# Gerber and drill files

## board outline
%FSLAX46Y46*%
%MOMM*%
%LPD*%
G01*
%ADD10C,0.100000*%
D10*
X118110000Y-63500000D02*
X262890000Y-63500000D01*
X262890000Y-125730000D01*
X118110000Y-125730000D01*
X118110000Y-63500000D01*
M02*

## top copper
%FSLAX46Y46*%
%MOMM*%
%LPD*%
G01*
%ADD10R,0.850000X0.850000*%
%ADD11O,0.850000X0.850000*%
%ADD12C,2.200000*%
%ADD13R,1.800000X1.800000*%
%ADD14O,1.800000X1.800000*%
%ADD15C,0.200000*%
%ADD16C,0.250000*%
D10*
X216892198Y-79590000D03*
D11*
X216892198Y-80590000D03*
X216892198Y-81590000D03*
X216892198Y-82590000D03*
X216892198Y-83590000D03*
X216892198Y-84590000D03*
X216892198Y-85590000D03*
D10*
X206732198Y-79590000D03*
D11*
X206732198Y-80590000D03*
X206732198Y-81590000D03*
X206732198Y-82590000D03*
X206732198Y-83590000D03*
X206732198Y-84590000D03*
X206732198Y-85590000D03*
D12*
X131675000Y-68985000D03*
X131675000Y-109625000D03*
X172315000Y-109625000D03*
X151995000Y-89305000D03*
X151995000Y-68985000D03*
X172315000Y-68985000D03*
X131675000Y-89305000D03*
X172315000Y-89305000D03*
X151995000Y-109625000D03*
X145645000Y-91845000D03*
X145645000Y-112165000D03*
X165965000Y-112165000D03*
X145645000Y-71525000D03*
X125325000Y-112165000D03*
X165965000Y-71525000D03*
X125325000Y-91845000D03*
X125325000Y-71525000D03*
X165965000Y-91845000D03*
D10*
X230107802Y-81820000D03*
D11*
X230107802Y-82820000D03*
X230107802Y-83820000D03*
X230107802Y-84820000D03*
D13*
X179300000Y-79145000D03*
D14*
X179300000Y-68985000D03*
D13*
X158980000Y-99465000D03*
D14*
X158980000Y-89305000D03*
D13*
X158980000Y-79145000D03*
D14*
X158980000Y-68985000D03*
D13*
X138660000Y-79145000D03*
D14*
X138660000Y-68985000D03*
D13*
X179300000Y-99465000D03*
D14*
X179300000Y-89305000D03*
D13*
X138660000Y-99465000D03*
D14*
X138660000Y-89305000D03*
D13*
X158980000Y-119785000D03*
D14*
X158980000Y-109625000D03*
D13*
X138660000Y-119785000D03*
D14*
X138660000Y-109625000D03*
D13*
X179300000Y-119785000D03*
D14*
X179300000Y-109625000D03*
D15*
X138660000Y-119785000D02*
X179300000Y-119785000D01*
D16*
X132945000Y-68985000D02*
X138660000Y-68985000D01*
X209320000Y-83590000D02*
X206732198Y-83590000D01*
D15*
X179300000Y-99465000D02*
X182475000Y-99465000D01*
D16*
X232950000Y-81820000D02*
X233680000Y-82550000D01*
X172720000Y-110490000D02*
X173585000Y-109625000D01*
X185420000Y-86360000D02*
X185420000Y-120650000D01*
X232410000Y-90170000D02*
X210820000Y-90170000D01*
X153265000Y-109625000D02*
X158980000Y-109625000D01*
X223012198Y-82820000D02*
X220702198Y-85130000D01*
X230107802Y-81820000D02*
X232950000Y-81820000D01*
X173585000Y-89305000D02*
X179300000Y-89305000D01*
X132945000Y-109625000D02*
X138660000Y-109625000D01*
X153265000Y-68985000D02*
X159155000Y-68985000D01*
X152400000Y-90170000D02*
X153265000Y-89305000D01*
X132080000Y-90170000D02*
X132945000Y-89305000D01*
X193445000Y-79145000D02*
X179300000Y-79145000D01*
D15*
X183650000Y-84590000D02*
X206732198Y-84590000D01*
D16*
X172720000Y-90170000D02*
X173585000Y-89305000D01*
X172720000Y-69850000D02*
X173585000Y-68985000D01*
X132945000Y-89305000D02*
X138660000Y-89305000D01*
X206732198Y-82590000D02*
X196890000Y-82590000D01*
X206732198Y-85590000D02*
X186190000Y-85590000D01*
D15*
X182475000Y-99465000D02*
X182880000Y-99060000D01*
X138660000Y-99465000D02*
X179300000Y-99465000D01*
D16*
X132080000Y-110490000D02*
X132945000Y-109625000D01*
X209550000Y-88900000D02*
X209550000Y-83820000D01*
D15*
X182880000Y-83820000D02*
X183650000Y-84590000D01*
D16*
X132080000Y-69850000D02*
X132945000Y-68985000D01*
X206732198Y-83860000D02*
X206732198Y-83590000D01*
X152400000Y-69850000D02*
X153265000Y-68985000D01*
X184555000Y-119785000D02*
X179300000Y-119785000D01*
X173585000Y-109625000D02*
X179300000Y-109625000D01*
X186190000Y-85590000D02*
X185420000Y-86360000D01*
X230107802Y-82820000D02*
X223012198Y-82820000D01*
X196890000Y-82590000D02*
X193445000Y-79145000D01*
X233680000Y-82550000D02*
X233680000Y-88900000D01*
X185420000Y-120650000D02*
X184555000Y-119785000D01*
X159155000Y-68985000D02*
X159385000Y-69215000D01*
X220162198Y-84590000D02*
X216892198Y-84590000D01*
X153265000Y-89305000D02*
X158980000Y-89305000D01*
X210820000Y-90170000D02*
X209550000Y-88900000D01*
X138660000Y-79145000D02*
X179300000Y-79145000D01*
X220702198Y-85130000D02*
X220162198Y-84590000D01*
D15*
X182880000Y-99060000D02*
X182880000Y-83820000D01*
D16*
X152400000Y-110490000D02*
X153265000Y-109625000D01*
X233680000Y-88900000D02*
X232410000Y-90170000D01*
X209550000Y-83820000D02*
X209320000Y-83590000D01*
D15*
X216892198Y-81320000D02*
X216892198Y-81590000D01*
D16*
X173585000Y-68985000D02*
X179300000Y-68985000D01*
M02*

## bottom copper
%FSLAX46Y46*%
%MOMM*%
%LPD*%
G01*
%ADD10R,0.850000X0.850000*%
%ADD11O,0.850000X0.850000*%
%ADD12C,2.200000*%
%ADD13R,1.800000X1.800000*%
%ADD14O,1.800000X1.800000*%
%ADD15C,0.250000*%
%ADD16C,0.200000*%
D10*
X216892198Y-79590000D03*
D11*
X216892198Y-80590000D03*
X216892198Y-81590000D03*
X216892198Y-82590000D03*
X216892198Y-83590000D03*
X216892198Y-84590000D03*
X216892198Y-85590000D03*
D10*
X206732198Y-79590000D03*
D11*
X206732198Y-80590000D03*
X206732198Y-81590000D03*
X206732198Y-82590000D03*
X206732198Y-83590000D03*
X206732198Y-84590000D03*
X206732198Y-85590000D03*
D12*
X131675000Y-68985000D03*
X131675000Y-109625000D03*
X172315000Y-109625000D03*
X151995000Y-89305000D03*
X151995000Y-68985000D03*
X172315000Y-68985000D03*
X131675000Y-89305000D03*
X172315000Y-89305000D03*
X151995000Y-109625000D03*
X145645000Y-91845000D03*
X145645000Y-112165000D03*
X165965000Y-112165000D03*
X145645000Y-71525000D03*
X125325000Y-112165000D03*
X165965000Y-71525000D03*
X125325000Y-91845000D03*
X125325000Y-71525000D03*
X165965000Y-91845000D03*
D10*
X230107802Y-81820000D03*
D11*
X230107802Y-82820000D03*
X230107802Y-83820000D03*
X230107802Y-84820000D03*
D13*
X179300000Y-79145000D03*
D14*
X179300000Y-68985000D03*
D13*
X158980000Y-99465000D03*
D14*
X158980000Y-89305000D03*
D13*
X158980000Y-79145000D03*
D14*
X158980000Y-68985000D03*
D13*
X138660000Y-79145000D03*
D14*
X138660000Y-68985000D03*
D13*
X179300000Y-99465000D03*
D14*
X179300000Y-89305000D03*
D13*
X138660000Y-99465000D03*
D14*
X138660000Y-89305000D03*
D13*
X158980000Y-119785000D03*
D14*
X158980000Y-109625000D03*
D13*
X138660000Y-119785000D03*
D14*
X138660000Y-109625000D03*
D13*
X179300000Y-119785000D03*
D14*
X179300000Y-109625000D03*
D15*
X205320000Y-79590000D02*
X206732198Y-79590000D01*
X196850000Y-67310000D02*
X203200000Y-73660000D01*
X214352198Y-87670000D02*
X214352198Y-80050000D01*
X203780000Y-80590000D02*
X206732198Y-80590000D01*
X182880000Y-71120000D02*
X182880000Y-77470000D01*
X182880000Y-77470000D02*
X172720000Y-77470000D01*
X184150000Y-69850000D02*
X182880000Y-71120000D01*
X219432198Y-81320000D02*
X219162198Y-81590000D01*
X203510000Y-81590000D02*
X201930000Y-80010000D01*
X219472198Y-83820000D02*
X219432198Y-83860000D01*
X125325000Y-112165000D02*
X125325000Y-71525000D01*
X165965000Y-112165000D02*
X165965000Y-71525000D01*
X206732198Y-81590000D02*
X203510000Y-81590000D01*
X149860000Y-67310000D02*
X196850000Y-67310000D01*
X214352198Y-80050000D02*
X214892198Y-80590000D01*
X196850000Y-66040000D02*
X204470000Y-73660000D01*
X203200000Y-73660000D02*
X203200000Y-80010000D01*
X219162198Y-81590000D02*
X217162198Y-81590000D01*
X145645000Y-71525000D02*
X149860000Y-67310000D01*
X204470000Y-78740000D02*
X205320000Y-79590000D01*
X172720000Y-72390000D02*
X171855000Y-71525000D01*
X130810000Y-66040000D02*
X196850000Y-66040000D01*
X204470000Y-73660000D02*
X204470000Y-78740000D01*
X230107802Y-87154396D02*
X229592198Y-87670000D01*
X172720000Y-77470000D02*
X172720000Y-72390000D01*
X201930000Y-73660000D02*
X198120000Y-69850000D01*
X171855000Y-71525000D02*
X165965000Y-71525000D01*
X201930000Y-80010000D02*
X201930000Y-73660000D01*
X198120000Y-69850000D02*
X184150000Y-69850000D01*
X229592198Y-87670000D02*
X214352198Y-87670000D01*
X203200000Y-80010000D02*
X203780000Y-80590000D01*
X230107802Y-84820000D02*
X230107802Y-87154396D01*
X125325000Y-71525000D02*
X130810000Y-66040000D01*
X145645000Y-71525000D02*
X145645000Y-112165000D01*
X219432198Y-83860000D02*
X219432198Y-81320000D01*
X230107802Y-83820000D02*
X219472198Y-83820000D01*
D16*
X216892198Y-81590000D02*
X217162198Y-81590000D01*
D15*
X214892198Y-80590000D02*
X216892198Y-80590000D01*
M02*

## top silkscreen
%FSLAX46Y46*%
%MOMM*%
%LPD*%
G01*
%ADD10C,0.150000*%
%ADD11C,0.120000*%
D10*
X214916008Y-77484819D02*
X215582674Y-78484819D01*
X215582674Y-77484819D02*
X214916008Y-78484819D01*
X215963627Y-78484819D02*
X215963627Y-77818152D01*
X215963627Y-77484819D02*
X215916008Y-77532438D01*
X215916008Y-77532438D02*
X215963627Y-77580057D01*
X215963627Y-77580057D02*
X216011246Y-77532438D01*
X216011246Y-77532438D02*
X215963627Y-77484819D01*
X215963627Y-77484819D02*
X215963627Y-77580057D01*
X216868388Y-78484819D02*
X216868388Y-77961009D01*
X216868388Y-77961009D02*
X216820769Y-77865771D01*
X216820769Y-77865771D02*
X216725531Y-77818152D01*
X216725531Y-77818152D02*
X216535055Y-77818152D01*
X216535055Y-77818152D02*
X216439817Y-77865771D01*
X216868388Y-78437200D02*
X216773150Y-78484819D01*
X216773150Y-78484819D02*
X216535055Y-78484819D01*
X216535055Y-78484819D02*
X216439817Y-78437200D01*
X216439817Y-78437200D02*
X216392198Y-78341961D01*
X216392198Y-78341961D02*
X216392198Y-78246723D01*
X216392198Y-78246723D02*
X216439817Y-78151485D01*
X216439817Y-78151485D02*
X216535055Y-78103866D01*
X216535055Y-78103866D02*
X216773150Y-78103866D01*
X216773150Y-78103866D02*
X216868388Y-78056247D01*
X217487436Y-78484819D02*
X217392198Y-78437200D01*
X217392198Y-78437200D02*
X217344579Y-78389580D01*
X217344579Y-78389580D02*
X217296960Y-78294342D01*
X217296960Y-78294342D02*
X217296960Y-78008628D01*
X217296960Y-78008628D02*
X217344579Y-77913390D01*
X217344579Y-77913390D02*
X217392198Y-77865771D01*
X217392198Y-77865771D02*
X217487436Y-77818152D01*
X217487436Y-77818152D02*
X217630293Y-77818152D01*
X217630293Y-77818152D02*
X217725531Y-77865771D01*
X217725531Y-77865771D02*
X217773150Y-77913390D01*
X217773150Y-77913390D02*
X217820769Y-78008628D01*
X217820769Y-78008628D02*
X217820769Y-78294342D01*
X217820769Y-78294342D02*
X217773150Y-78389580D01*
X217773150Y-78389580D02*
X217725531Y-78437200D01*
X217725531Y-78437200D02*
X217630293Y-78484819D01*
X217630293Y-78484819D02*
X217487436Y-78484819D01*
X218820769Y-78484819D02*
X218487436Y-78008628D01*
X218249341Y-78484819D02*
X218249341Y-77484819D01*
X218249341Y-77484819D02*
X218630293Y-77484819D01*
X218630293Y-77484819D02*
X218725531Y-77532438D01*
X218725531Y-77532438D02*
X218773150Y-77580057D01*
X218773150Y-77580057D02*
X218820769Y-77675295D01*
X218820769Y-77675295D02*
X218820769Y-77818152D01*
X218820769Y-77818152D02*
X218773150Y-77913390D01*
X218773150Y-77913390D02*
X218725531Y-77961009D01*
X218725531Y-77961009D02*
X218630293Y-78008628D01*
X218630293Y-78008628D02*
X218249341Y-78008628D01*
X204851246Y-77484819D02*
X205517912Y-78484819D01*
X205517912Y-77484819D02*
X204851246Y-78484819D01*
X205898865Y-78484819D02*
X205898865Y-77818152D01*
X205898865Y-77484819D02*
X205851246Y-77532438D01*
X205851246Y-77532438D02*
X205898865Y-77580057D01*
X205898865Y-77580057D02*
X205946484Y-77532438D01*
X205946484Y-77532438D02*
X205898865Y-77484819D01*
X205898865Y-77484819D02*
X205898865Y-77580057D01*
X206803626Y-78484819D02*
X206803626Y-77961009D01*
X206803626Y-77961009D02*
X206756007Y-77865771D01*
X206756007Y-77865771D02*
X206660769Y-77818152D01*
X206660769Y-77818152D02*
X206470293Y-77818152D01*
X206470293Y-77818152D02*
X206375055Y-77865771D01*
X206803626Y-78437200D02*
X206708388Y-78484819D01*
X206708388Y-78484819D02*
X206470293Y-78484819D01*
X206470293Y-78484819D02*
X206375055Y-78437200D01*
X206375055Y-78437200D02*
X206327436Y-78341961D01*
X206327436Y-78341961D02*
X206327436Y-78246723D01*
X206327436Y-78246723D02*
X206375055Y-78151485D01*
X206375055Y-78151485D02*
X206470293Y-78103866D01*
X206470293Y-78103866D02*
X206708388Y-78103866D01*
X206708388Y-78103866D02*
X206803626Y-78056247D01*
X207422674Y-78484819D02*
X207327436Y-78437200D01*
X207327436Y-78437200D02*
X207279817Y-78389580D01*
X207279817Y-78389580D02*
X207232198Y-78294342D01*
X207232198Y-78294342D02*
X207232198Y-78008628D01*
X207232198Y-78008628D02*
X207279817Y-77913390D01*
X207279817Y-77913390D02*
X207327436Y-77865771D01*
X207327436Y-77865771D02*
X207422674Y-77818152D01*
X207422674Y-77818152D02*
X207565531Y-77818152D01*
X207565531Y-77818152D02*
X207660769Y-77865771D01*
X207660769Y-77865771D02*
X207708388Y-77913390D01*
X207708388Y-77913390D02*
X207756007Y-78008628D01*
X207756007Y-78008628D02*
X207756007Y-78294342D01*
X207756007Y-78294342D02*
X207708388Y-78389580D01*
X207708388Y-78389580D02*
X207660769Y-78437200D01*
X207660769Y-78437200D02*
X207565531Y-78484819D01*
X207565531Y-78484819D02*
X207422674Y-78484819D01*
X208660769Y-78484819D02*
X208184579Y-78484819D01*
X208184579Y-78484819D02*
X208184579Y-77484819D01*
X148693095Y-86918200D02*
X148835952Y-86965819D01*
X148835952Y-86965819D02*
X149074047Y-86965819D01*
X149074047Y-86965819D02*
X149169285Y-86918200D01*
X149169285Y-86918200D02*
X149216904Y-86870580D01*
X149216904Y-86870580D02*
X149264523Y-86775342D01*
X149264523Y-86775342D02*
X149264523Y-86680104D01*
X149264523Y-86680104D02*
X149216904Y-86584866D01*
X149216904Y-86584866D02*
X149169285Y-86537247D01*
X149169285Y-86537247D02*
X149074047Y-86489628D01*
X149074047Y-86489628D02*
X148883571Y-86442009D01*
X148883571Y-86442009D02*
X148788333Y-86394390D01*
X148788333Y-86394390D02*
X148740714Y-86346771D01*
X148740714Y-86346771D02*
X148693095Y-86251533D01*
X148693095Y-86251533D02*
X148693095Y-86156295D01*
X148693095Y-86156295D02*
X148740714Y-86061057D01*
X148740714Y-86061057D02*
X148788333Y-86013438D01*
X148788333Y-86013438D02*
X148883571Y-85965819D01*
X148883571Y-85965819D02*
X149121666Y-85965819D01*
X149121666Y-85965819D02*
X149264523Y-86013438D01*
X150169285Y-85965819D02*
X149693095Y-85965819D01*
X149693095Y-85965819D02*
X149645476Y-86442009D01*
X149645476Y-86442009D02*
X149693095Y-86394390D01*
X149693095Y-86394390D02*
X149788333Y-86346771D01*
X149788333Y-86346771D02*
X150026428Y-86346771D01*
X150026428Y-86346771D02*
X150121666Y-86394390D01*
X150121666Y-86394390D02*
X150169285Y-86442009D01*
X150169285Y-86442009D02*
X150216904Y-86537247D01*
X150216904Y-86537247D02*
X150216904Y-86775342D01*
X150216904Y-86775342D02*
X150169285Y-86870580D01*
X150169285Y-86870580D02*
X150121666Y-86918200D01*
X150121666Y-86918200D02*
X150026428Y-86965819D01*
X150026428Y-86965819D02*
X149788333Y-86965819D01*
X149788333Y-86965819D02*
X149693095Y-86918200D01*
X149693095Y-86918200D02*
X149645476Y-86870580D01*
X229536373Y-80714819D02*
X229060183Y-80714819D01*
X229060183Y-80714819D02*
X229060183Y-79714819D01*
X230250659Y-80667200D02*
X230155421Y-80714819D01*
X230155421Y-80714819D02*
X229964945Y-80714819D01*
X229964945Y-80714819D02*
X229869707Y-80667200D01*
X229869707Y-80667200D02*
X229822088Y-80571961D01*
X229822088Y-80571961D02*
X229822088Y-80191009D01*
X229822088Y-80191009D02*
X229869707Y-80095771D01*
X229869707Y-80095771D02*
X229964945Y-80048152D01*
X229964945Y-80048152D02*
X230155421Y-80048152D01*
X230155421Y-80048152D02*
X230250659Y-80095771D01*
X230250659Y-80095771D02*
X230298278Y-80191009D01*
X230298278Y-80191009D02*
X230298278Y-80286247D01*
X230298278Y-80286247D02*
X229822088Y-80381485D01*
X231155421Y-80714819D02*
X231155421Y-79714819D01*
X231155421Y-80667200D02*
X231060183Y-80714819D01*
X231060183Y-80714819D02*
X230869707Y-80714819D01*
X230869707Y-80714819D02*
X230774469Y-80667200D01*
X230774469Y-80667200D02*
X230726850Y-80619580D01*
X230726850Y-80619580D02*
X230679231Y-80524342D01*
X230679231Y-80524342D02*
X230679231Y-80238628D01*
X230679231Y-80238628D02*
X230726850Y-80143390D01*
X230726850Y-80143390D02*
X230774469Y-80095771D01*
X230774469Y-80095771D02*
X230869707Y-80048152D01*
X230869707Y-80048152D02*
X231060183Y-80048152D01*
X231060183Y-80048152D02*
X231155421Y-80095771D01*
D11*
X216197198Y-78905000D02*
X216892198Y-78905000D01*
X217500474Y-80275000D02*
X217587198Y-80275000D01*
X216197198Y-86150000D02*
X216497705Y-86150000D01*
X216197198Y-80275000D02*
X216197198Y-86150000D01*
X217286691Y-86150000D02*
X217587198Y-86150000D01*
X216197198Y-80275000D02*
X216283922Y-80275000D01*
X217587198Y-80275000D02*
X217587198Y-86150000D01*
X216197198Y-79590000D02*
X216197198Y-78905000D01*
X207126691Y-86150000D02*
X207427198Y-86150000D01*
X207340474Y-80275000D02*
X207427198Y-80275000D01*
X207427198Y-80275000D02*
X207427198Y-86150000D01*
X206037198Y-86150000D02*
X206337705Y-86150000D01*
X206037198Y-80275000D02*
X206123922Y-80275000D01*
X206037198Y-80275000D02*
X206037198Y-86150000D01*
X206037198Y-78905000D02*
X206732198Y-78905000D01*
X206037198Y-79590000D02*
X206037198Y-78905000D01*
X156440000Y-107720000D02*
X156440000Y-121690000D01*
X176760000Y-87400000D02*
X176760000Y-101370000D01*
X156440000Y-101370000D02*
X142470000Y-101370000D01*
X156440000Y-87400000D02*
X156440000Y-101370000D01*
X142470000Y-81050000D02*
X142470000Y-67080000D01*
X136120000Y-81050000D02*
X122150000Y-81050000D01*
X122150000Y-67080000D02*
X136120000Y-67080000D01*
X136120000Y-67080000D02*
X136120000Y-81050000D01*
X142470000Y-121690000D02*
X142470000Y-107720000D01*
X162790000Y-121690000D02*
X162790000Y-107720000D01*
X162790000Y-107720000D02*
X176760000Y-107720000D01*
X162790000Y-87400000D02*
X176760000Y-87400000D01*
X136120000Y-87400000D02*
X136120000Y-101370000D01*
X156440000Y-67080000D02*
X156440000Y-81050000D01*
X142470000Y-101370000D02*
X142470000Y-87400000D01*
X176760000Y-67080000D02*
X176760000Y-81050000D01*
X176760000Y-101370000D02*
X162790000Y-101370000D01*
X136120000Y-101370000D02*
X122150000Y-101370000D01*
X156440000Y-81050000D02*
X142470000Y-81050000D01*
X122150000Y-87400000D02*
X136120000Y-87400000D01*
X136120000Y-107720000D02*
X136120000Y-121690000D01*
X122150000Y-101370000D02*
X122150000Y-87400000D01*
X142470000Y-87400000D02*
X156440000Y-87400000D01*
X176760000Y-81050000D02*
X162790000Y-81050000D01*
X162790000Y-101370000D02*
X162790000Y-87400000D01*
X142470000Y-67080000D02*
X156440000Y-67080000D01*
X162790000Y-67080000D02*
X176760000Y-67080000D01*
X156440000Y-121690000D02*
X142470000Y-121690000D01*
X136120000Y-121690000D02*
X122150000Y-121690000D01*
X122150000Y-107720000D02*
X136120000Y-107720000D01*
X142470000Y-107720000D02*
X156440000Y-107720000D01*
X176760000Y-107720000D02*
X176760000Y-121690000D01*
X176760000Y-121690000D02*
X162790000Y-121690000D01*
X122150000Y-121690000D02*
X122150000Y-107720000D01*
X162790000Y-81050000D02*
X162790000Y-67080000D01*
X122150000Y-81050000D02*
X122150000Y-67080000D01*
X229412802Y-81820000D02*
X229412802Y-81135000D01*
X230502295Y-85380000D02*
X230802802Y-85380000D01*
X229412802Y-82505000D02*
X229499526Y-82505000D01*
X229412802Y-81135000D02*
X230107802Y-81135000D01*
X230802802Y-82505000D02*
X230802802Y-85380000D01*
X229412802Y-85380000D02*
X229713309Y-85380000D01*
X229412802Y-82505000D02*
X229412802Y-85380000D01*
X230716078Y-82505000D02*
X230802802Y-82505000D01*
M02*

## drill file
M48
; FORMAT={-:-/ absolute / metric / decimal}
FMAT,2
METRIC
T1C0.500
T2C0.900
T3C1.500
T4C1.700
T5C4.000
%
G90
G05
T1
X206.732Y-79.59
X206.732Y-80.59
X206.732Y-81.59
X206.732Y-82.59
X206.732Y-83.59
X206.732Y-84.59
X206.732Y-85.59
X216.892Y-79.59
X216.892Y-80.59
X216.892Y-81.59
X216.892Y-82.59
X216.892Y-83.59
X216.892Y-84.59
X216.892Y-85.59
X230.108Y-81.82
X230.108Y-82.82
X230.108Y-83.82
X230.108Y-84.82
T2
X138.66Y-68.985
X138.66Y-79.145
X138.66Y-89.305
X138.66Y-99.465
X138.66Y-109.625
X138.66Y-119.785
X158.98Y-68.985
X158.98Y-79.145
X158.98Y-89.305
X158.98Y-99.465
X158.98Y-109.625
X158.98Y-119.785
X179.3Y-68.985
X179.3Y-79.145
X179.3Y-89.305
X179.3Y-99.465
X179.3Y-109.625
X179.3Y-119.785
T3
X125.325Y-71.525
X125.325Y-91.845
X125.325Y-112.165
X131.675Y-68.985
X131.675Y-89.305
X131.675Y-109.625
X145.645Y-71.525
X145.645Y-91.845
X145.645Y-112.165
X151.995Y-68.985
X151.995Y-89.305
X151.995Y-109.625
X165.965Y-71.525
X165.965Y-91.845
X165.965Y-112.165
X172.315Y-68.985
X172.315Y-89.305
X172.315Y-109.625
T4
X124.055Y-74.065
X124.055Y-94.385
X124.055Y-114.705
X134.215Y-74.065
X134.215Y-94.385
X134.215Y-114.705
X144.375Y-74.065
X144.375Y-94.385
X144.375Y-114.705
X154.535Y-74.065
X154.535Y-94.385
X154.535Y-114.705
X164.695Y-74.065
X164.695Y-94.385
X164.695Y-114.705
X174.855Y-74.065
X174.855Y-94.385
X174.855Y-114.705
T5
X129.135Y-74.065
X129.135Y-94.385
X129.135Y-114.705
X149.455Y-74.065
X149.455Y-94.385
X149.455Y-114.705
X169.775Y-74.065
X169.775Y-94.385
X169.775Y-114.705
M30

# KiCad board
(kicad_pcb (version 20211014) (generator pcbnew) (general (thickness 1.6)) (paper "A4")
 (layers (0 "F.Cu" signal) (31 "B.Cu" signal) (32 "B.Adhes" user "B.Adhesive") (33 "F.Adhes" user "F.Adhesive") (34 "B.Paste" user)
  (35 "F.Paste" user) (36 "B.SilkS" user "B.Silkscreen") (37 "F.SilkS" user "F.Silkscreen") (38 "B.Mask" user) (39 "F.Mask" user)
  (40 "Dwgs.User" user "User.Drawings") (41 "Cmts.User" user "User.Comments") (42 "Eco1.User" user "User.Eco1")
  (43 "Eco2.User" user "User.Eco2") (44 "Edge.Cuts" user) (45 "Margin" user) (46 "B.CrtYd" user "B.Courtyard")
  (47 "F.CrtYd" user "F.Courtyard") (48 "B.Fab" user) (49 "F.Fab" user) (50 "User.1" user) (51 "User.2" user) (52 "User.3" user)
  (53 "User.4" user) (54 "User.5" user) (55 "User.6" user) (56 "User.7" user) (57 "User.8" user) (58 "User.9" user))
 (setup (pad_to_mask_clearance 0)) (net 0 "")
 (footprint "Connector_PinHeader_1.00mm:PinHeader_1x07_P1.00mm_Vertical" (layer "F.Cu") (at 216.892198 79.59)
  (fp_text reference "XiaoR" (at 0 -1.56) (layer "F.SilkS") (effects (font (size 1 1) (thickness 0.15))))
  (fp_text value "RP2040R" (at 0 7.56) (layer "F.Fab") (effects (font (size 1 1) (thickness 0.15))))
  (fp_line (start -0.695 -0.685) (end 0 -0.685) (layer "F.SilkS") (width 0.12))
  (fp_line (start 0.608276 0.685) (end 0.695 0.685) (layer "F.SilkS") (width 0.12))
  (fp_line (start -0.695 6.56) (end -0.394493 6.56) (layer "F.SilkS") (width 0.12))
  (fp_line (start -0.695 0.685) (end -0.695 6.56) (layer "F.SilkS") (width 0.12))
  (fp_line (start 0.394493 6.56) (end 0.695 6.56) (layer "F.SilkS") (width 0.12))
  (fp_line (start -0.695 0.685) (end -0.608276 0.685) (layer "F.SilkS") (width 0.12))
  (fp_line (start 0.695 0.685) (end 0.695 6.56) (layer "F.SilkS") (width 0.12))
  (fp_line (start -0.695 0) (end -0.695 -0.685) (layer "F.SilkS") (width 0.12))
  (pad "1" thru_hole rect (at 0 0) (size 0.85 0.85) (drill 0.5) (layers F&B.Cu *.Mask))
  (pad "2" thru_hole oval (at 0 1) (size 0.85 0.85) (drill 0.5) (layers F&B.Cu *.Mask))
  (pad "3" thru_hole oval (at 0 2) (size 0.85 0.85) (drill 0.5) (layers F&B.Cu *.Mask))
  (pad "4" thru_hole oval (at 0 3) (size 0.85 0.85) (drill 0.5) (layers F&B.Cu *.Mask))
  (pad "5" thru_hole oval (at 0 4) (size 0.85 0.85) (drill 0.5) (layers F&B.Cu *.Mask))
  (pad "6" thru_hole oval (at 0 5) (size 0.85 0.85) (drill 0.5) (layers F&B.Cu *.Mask))
  (pad "7" thru_hole oval (at 0 6) (size 0.85 0.85) (drill 0.5) (layers F&B.Cu *.Mask)))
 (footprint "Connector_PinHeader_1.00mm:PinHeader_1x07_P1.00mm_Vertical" (layer "F.Cu") (at 206.732198 79.59)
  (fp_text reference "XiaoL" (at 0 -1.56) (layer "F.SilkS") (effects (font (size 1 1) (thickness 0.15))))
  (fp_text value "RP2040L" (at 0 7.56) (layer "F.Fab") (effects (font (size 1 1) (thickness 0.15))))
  (fp_line (start 0.394493 6.56) (end 0.695 6.56) (layer "F.SilkS") (width 0.12))
  (fp_line (start 0.608276 0.685) (end 0.695 0.685) (layer "F.SilkS") (width 0.12))
  (fp_line (start 0.695 0.685) (end 0.695 6.56) (layer "F.SilkS") (width 0.12))
  (fp_line (start -0.695 6.56) (end -0.394493 6.56) (layer "F.SilkS") (width 0.12))
  (fp_line (start -0.695 0.685) (end -0.608276 0.685) (layer "F.SilkS") (width 0.12))
  (fp_line (start -0.695 0.685) (end -0.695 6.56) (layer "F.SilkS") (width 0.12))
  (fp_line (start -0.695 -0.685) (end 0 -0.685) (layer "F.SilkS") (width 0.12))
  (fp_line (start -0.695 0) (end -0.695 -0.685) (layer "F.SilkS") (width 0.12))
  (pad "1" thru_hole rect (at 0 0) (size 0.85 0.85) (drill 0.5) (layers *.Cu *.Mask))
  (pad "2" thru_hole oval (at 0 1) (size 0.85 0.85) (drill 0.5) (layers *.Cu *.Mask))
  (pad "3" thru_hole oval (at 0 2) (size 0.85 0.85) (drill 0.5) (layers *.Cu *.Mask))
  (pad "4" thru_hole oval (at 0 3) (size 0.85 0.85) (drill 0.5) (layers *.Cu *.Mask))
  (pad "5" thru_hole oval (at 0 4) (size 0.85 0.85) (drill 0.5) (layers *.Cu *.Mask))
  (pad "6" thru_hole oval (at 0 5) (size 0.85 0.85) (drill 0.5) (layers *.Cu *.Mask))
  (pad "7" thru_hole oval (at 0 6) (size 0.85 0.85) (drill 0.5) (layers *.Cu *.Mask)))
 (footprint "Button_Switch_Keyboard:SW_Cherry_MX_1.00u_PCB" (layer "F.Cu") (at 276.455 61.365)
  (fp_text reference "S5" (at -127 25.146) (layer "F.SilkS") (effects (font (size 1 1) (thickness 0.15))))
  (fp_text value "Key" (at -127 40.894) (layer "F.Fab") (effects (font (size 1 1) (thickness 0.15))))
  (fp_line (start -120.015 46.355) (end -120.015 60.325) (layer "F.SilkS") (width 0.12))
  (fp_line (start -99.695 26.035) (end -99.695 40.005) (layer "F.SilkS") (width 0.12))
  (fp_line (start -120.015 40.005) (end -133.985 40.005) (layer "F.SilkS") (width 0.12))
  (fp_line (start -120.015 26.035) (end -120.015 40.005) (layer "F.SilkS") (width 0.12))
  (fp_line (start -133.985 19.685) (end -133.985 5.715) (layer "F.SilkS") (width 0.12))
  (fp_line (start -140.335 19.685) (end -154.305 19.685) (layer "F.SilkS") (width 0.12))
  (fp_line (start -154.305 5.715) (end -140.335 5.715) (layer "F.SilkS") (width 0.12))
  (fp_line (start -140.335 5.715) (end -140.335 19.685) (layer "F.SilkS") (width 0.12))
  (fp_line (start -133.985 60.325) (end -133.985 46.355) (layer "F.SilkS") (width 0.12))
  (fp_line (start -113.665 60.325) (end -113.665 46.355) (layer "F.SilkS") (width 0.12))
  (fp_line (start -113.665 46.355) (end -99.695 46.355) (layer "F.SilkS") (width 0.12))
  (fp_line (start -113.665 26.035) (end -99.695 26.035) (layer "F.SilkS") (width 0.12))
  (fp_line (start -140.335 26.035) (end -140.335 40.005) (layer "F.SilkS") (width 0.12))
  (fp_line (start -120.015 5.715) (end -120.015 19.685) (layer "F.SilkS") (width 0.12))
  (fp_line (start -133.985 40.005) (end -133.985 26.035) (layer "F.SilkS") (width 0.12))
  (fp_line (start -99.695 5.715) (end -99.695 19.685) (layer "F.SilkS") (width 0.12))
  (fp_line (start -99.695 40.005) (end -113.665 40.005) (layer "F.SilkS") (width 0.12))
  (fp_line (start -140.335 40.005) (end -154.305 40.005) (layer "F.SilkS") (width 0.12))
  (fp_line (start -120.015 19.685) (end -133.985 19.685) (layer "F.SilkS") (width 0.12))
  (fp_line (start -154.305 26.035) (end -140.335 26.035) (layer "F.SilkS") (width 0.12))
  (fp_line (start -140.335 46.355) (end -140.335 60.325) (layer "F.SilkS") (width 0.12))
  (fp_line (start -154.305 40.005) (end -154.305 26.035) (layer "F.SilkS") (width 0.12))
  (fp_line (start -133.985 26.035) (end -120.015 26.035) (layer "F.SilkS") (width 0.12))
  (fp_line (start -99.695 19.685) (end -113.665 19.685) (layer "F.SilkS") (width 0.12))
  (fp_line (start -113.665 40.005) (end -113.665 26.035) (layer "F.SilkS") (width 0.12))
  (fp_line (start -133.985 5.715) (end -120.015 5.715) (layer "F.SilkS") (width 0.12))
  (fp_line (start -113.665 5.715) (end -99.695 5.715) (layer "F.SilkS") (width 0.12))
  (fp_line (start -120.015 60.325) (end -133.985 60.325) (layer "F.SilkS") (width 0.12))
  (fp_line (start -140.335 60.325) (end -154.305 60.325) (layer "F.SilkS") (width 0.12))
  (fp_line (start -154.305 46.355) (end -140.335 46.355) (layer "F.SilkS") (width 0.12))
  (fp_line (start -133.985 46.355) (end -120.015 46.355) (layer "F.SilkS") (width 0.12))
  (fp_line (start -99.695 46.355) (end -99.695 60.325) (layer "F.SilkS") (width 0.12))
  (fp_line (start -99.695 60.325) (end -113.665 60.325) (layer "F.SilkS") (width 0.12))
  (fp_line (start -154.305 60.325) (end -154.305 46.355) (layer "F.SilkS") (width 0.12))
  (fp_line (start -113.665 19.685) (end -113.665 5.715) (layer "F.SilkS") (width 0.12))
  (fp_line (start -154.305 19.685) (end -154.305 5.715) (layer "F.SilkS") (width 0.12))
  (pad "" np_thru_hole circle (at -152.4 33.02) (size 1.7 1.7) (drill 1.7) (layers *.Cu *.Mask))
  (pad "" np_thru_hole circle (at -121.92 53.34) (size 1.7 1.7) (drill 1.7) (layers *.Cu *.Mask))
  (pad "" np_thru_hole circle (at -132.08 12.7) (size 1.7 1.7) (drill 1.7) (layers *.Cu *.Mask))
  (pad "" np_thru_hole circle (at -127 33.02) (size 4 4) (drill 4) (layers *.Cu *.Mask))
  (pad "" np_thru_hole circle (at -142.24 12.7) (size 1.7 1.7) (drill 1.7) (layers *.Cu *.Mask))
  (pad "" np_thru_hole circle (at -147.32 53.34) (size 4 4) (drill 4) (layers *.Cu *.Mask))
  (pad "" np_thru_hole circle (at -152.4 12.7) (size 1.7 1.7) (drill 1.7) (layers *.Cu *.Mask))
  (pad "" np_thru_hole circle (at -106.68 12.7) (size 4 4) (drill 4) (layers *.Cu *.Mask))
  (pad "" np_thru_hole circle (at -142.24 33.02) (size 1.7 1.7) (drill 1.7) (layers *.Cu *.Mask))
  (pad "" np_thru_hole circle (at -127 53.34) (size 4 4) (drill 4) (layers *.Cu *.Mask))
  (pad "" np_thru_hole circle (at -111.76 53.34) (size 1.7 1.7) (drill 1.7) (layers *.Cu *.Mask))
  (pad "" np_thru_hole circle (at -127 12.7) (size 4 4) (drill 4) (layers *.Cu *.Mask))
  (pad "" np_thru_hole circle (at -142.24 53.34) (size 1.7 1.7) (drill 1.7) (layers *.Cu *.Mask))
  (pad "" np_thru_hole circle (at -147.32 12.7) (size 4 4) (drill 4) (layers *.Cu *.Mask))
  (pad "" np_thru_hole circle (at -132.08 53.34) (size 1.7 1.7) (drill 1.7) (layers *.Cu *.Mask))
  (pad "" np_thru_hole circle (at -101.6 53.34) (size 1.7 1.7) (drill 1.7) (layers *.Cu *.Mask))
  (pad "" np_thru_hole circle (at -106.68 33.02) (size 4 4) (drill 4) (layers *.Cu *.Mask))
  (pad "" np_thru_hole circle (at -101.6 33.02) (size 1.7 1.7) (drill 1.7) (layers *.Cu *.Mask))
  (pad "" np_thru_hole circle (at -101.6 12.7) (size 1.7 1.7) (drill 1.7) (layers *.Cu *.Mask))
  (pad "" np_thru_hole circle (at -121.92 12.7) (size 1.7 1.7) (drill 1.7) (layers *.Cu *.Mask))
  (pad "" np_thru_hole circle (at -111.76 33.02) (size 1.7 1.7) (drill 1.7) (layers *.Cu *.Mask))
  (pad "" np_thru_hole circle (at -121.92 33.02) (size 1.7 1.7) (drill 1.7) (layers *.Cu *.Mask))
  (pad "" np_thru_hole circle (at -106.68 53.34) (size 4 4) (drill 4) (layers *.Cu *.Mask))
  (pad "" np_thru_hole circle (at -152.4 53.34) (size 1.7 1.7) (drill 1.7) (layers *.Cu *.Mask))
  (pad "" np_thru_hole circle (at -111.76 12.7) (size 1.7 1.7) (drill 1.7) (layers *.Cu *.Mask))
  (pad "" np_thru_hole circle (at -147.32 33.02) (size 4 4) (drill 4) (layers *.Cu *.Mask))
  (pad "" np_thru_hole circle (at -132.08 33.02) (size 1.7 1.7) (drill 1.7) (layers *.Cu *.Mask))
  (pad "1" thru_hole circle (at -144.78 7.62) (size 2.2 2.2) (drill 1.5) (layers *.Cu *.Mask))
  (pad "1" thru_hole circle (at -144.78 48.26) (size 2.2 2.2) (drill 1.5) (layers *.Cu *.Mask))
  (pad "1" thru_hole circle (at -104.14 48.26) (size 2.2 2.2) (drill 1.5) (layers *.Cu *.Mask))
  (pad "1" thru_hole circle (at -124.46 27.94) (size 2.2 2.2) (drill 1.5) (layers *.Cu *.Mask))
  (pad "1" thru_hole circle (at -124.46 7.62) (size 2.2 2.2) (drill 1.5) (layers *.Cu *.Mask))
  (pad "1" thru_hole circle (at -104.14 7.62) (size 2.2 2.2) (drill 1.5) (layers *.Cu *.Mask))
  (pad "1" thru_hole circle (at -144.78 27.94) (size 2.2 2.2) (drill 1.5) (layers *.Cu *.Mask))
  (pad "1" thru_hole circle (at -104.14 27.94) (size 2.2 2.2) (drill 1.5) (layers *.Cu *.Mask))
  (pad "1" thru_hole circle (at -124.46 48.26) (size 2.2 2.2) (drill 1.5) (layers *.Cu *.Mask))
  (pad "2" thru_hole circle (at -130.81 30.48) (size 2.2 2.2) (drill 1.5) (layers *.Cu *.Mask))
  (pad "2" thru_hole circle (at -130.81 50.8) (size 2.2 2.2) (drill 1.5) (layers *.Cu *.Mask))
  (pad "2" thru_hole circle (at -110.49 50.8) (size 2.2 2.2) (drill 1.5) (layers *.Cu *.Mask))
  (pad "2" thru_hole circle (at -130.81 10.16) (size 2.2 2.2) (drill 1.5) (layers *.Cu *.Mask))
  (pad "2" thru_hole circle (at -151.13 50.8) (size 2.2 2.2) (drill 1.5) (layers *.Cu *.Mask))
  (pad "2" thru_hole circle (at -110.49 10.16) (size 2.2 2.2) (drill 1.5) (layers *.Cu *.Mask))
  (pad "2" thru_hole circle (at -151.13 30.48) (size 2.2 2.2) (drill 1.5) (layers *.Cu *.Mask))
  (pad "2" thru_hole circle (at -151.13 10.16) (size 2.2 2.2) (drill 1.5) (layers *.Cu *.Mask))
  (pad "2" thru_hole circle (at -110.49 30.48) (size 2.2 2.2) (drill 1.5) (layers *.Cu *.Mask)))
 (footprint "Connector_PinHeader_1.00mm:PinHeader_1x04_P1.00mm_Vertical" (layer "F.Cu") (at 230.107802 81.82)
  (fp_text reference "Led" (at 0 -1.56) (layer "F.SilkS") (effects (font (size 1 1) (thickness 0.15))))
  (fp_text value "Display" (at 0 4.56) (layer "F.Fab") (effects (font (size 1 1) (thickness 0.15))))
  (fp_line (start -0.695 0) (end -0.695 -0.685) (layer "F.SilkS") (width 0.12))
  (fp_line (start 0.394493 3.56) (end 0.695 3.56) (layer "F.SilkS") (width 0.12))
  (fp_line (start -0.695 0.685) (end -0.608276 0.685) (layer "F.SilkS") (width 0.12))
  (fp_line (start -0.695 -0.685) (end 0 -0.685) (layer "F.SilkS") (width 0.12))
  (fp_line (start 0.695 0.685) (end 0.695 3.56) (layer "F.SilkS") (width 0.12))
  (fp_line (start -0.695 3.56) (end -0.394493 3.56) (layer "F.SilkS") (width 0.12))
  (fp_line (start -0.695 0.685) (end -0.695 3.56) (layer "F.SilkS") (width 0.12))
  (fp_line (start 0.608276 0.685) (end 0.695 0.685) (layer "F.SilkS") (width 0.12))
  (pad "1" thru_hole rect (at 0 0) (size 0.85 0.85) (drill 0.5) (layers *.Cu *.Mask))
  (pad "2" thru_hole oval (at 0 1) (size 0.85 0.85) (drill 0.5) (layers *.Cu *.Mask))
  (pad "3" thru_hole oval (at 0 2) (size 0.85 0.85) (drill 0.5) (layers *.Cu *.Mask))
  (pad "4" thru_hole oval (at 0 3) (size 0.85 0.85) (drill 0.5) (layers *.Cu *.Mask)))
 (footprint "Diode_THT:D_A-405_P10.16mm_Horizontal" (layer "B.Cu") (at 179.3 79.145 90)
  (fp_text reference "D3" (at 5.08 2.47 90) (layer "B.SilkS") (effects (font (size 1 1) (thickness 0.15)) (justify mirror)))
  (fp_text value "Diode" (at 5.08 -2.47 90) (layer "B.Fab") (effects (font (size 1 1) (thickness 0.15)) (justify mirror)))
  (pad "1" thru_hole rect (at 0 0 90) (size 1.8 1.8) (drill 0.9) (layers F&B.Cu *.Mask))
  (pad "2" thru_hole oval (at 10.16 0 90) (size 1.8 1.8) (drill 0.9) (layers F&B.Cu *.Mask)))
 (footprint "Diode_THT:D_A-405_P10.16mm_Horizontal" (layer "B.Cu") (at 158.98 99.465 90)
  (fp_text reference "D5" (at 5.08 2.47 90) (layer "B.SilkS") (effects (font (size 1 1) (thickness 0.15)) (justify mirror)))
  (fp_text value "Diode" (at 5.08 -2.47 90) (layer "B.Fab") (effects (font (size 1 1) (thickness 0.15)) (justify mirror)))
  (pad "1" thru_hole rect (at 0 0 90) (size 1.8 1.8) (drill 0.9) (layers F&B.Cu *.Mask))
  (pad "2" thru_hole oval (at 10.16 0 90) (size 1.8 1.8) (drill 0.9) (layers F&B.Cu *.Mask)))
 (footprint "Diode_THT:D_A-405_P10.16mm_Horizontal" (layer "B.Cu") (at 158.98 79.145 90)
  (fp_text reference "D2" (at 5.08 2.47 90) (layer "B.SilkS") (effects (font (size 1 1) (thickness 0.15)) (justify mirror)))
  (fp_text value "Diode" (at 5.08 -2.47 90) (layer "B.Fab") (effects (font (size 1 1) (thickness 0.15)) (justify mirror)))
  (pad "1" thru_hole rect (at 0 0 90) (size 1.8 1.8) (drill 0.9) (layers F&B.Cu *.Mask))
  (pad "2" thru_hole oval (at 10.16 0 90) (size 1.8 1.8) (drill 0.9) (layers F&B.Cu *.Mask)))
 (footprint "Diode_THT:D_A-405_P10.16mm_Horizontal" (layer "B.Cu") (at 138.66 79.145 90)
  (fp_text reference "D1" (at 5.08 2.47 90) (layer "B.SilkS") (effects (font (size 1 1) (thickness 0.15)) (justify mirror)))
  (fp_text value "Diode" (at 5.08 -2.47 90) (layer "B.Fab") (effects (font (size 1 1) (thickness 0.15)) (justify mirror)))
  (pad "1" thru_hole rect (at 0 0 90) (size 1.8 1.8) (drill 0.9) (layers *.Cu *.Mask))
  (pad "2" thru_hole oval (at 10.16 0 90) (size 1.8 1.8) (drill 0.9) (layers *.Cu *.Mask)))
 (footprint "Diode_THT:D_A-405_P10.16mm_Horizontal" (layer "B.Cu") (at 179.3 99.465 90)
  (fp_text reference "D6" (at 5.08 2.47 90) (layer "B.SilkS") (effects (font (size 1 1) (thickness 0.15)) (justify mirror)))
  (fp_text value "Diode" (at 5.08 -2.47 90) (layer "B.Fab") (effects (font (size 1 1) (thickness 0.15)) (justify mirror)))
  (pad "1" thru_hole rect (at 0 0 90) (size 1.8 1.8) (drill 0.9) (layers F&B.Cu *.Mask))
  (pad "2" thru_hole oval (at 10.16 0 90) (size 1.8 1.8) (drill 0.9) (layers F&B.Cu *.Mask)))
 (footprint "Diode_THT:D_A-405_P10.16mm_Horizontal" (layer "B.Cu") (at 138.66 99.465 90)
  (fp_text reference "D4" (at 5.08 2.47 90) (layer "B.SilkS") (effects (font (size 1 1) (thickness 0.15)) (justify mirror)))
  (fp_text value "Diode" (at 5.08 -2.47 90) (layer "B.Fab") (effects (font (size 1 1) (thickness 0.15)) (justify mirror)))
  (pad "1" thru_hole rect (at 0 0 90) (size 1.8 1.8) (drill 0.9) (layers F&B.Cu *.Mask))
  (pad "2" thru_hole oval (at 10.16 0 90) (size 1.8 1.8) (drill 0.9) (layers F&B.Cu *.Mask)))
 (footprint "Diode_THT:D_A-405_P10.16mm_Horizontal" (layer "B.Cu") (at 158.98 119.785 90)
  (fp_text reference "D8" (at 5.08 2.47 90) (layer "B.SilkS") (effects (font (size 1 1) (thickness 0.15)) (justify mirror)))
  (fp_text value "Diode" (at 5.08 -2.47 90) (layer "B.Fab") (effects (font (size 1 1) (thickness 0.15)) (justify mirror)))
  (pad "1" thru_hole rect (at 0 0 90) (size 1.8 1.8) (drill 0.9) (layers F&B.Cu *.Mask))
  (pad "2" thru_hole oval (at 10.16 0 90) (size 1.8 1.8) (drill 0.9) (layers F&B.Cu *.Mask)))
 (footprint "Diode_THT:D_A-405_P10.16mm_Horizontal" (layer "B.Cu") (at 138.66 119.785 90)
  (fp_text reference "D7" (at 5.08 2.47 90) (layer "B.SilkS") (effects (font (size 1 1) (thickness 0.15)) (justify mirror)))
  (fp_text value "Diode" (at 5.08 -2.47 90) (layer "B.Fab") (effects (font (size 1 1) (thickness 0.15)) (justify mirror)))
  (pad "1" thru_hole rect (at 0 0 90) (size 1.8 1.8) (drill 0.9) (layers F&B.Cu *.Mask))
  (pad "2" thru_hole oval (at 10.16 0 90) (size 1.8 1.8) (drill 0.9) (layers F&B.Cu *.Mask)))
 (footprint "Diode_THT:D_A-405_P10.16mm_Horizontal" (layer "B.Cu") (at 179.3 119.785 90)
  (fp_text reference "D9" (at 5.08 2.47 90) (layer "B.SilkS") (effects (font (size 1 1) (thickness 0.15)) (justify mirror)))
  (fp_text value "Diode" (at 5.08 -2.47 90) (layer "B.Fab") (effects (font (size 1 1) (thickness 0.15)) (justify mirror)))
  (pad "1" thru_hole rect (at 0 0 90) (size 1.8 1.8) (drill 0.9) (layers F&B.Cu *.Mask))
  (pad "2" thru_hole oval (at 10.16 0 90) (size 1.8 1.8) (drill 0.9) (layers F&B.Cu *.Mask)))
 (gr_rect (start 262.89 125.73) (end 118.11 63.5) (layer "Edge.Cuts") (width 0.1) (fill none))
 (segment (start 138.66 119.785) (end 179.3 119.785) (width 0.2) (layer "F.Cu") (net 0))
 (segment (start 132.945 68.985) (end 138.66 68.985) (width 0.25) (layer "F.Cu") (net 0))
 (segment (start 209.32 83.59) (end 206.732198 83.59) (width 0.25) (layer "F.Cu") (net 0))
 (segment (start 179.3 99.465) (end 182.475 99.465) (width 0.2) (layer "F.Cu") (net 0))
 (segment (start 232.95 81.82) (end 233.68 82.55) (width 0.25) (layer "F.Cu") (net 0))
 (segment (start 172.72 110.49) (end 173.585 109.625) (width 0.25) (layer "F.Cu") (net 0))
 (segment (start 185.42 86.36) (end 185.42 120.65) (width 0.25) (layer "F.Cu") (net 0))
 (segment (start 232.41 90.17) (end 210.82 90.17) (width 0.25) (layer "F.Cu") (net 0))
 (segment (start 153.265 109.625) (end 158.98 109.625) (width 0.25) (layer "F.Cu") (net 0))
 (segment (start 223.012198 82.82) (end 220.702198 85.13) (width 0.25) (layer "F.Cu") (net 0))
 (segment (start 230.107802 81.82) (end 232.95 81.82) (width 0.25) (layer "F.Cu") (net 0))
 (segment (start 173.585 89.305) (end 179.3 89.305) (width 0.25) (layer "F.Cu") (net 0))
 (segment (start 132.945 109.625) (end 138.66 109.625) (width 0.25) (layer "F.Cu") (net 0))
 (segment (start 153.265 68.985) (end 159.155 68.985) (width 0.25) (layer "F.Cu") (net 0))
 (segment (start 152.4 90.17) (end 153.265 89.305) (width 0.25) (layer "F.Cu") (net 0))
 (segment (start 132.08 90.17) (end 132.945 89.305) (width 0.25) (layer "F.Cu") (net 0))
 (segment (start 193.445 79.145) (end 179.3 79.145) (width 0.25) (layer "F.Cu") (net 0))
 (segment (start 183.65 84.59) (end 206.732198 84.59) (width 0.2) (layer "F.Cu") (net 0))
 (segment (start 172.72 90.17) (end 173.585 89.305) (width 0.25) (layer "F.Cu") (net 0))
 (segment (start 172.72 69.85) (end 173.585 68.985) (width 0.25) (layer "F.Cu") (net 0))
 (segment (start 132.945 89.305) (end 138.66 89.305) (width 0.25) (layer "F.Cu") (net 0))
 (segment (start 206.732198 82.59) (end 196.89 82.59) (width 0.25) (layer "F.Cu") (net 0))
 (segment (start 206.732198 85.59) (end 186.19 85.59) (width 0.25) (layer "F.Cu") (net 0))
 (segment (start 182.475 99.465) (end 182.88 99.06) (width 0.2) (layer "F.Cu") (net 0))
 (segment (start 138.66 99.465) (end 179.3 99.465) (width 0.2) (layer "F.Cu") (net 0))
 (segment (start 132.08 110.49) (end 132.945 109.625) (width 0.25) (layer "F.Cu") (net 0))
 (segment (start 209.55 88.9) (end 209.55 83.82) (width 0.25) (layer "F.Cu") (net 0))
 (segment (start 182.88 83.82) (end 183.65 84.59) (width 0.2) (layer "F.Cu") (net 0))
 (segment (start 132.08 69.85) (end 132.945 68.985) (width 0.25) (layer "F.Cu") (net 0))
 (segment (start 206.732198 83.86) (end 206.732198 83.59) (width 0.25) (layer "F.Cu") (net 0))
 (segment (start 152.4 69.85) (end 153.265 68.985) (width 0.25) (layer "F.Cu") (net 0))
 (segment (start 184.555 119.785) (end 179.3 119.785) (width 0.25) (layer "F.Cu") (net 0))
 (segment (start 173.585 109.625) (end 179.3 109.625) (width 0.25) (layer "F.Cu") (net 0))
 (segment (start 186.19 85.59) (end 185.42 86.36) (width 0.25) (layer "F.Cu") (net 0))
 (segment locked (start 230.107802 82.82) (end 223.012198 82.82) (width 0.25) (layer "F.Cu") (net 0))
 (segment (start 196.89 82.59) (end 193.445 79.145) (width 0.25) (layer "F.Cu") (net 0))
 (segment (start 233.68 82.55) (end 233.68 88.9) (width 0.25) (layer "F.Cu") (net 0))
 (segment (start 185.42 120.65) (end 184.555 119.785) (width 0.25) (layer "F.Cu") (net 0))
 (segment (start 159.155 68.985) (end 159.385 69.215) (width 0.25) (layer "F.Cu") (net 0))
 (segment (start 220.162198 84.59) (end 216.892198 84.59) (width 0.25) (layer "F.Cu") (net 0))
 (segment (start 153.265 89.305) (end 158.98 89.305) (width 0.25) (layer "F.Cu") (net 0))
 (segment (start 210.82 90.17) (end 209.55 88.9) (width 0.25) (layer "F.Cu") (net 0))
 (segment (start 138.66 79.145) (end 179.3 79.145) (width 0.25) (layer "F.Cu") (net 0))
 (segment (start 220.702198 85.13) (end 220.162198 84.59) (width 0.25) (layer "F.Cu") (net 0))
 (segment (start 182.88 99.06) (end 182.88 83.82) (width 0.2) (layer "F.Cu") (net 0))
 (segment (start 152.4 110.49) (end 153.265 109.625) (width 0.25) (layer "F.Cu") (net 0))
 (segment (start 233.68 88.9) (end 232.41 90.17) (width 0.25) (layer "F.Cu") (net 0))
 (segment (start 209.55 83.82) (end 209.32 83.59) (width 0.25) (layer "F.Cu") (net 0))
 (segment (start 216.892198 81.32) (end 216.892198 81.59) (width 0.2) (layer "F.Cu") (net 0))
 (segment (start 173.585 68.985) (end 179.3 68.985) (width 0.25) (layer "F.Cu") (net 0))
 (segment (start 205.32 79.59) (end 206.732198 79.59) (width 0.25) (layer "B.Cu") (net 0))
 (segment (start 196.85 67.31) (end 203.2 73.66) (width 0.25) (layer "B.Cu") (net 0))
 (segment (start 214.352198 87.67) (end 214.352198 80.05) (width 0.25) (layer "B.Cu") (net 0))
 (segment (start 203.78 80.59) (end 206.732198 80.59) (width 0.25) (layer "B.Cu") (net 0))
 (segment (start 182.88 71.12) (end 182.88 77.47) (width 0.25) (layer "B.Cu") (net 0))
 (segment (start 182.88 77.47) (end 172.72 77.47) (width 0.25) (layer "B.Cu") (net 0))
 (segment (start 184.15 69.85) (end 182.88 71.12) (width 0.25) (layer "B.Cu") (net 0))
 (segment (start 219.432198 81.32) (end 219.162198 81.59) (width 0.25) (layer "B.Cu") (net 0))
 (segment (start 203.51 81.59) (end 201.93 80.01) (width 0.25) (layer "B.Cu") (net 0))
 (segment (start 219.472198 83.82) (end 219.432198 83.86) (width 0.25) (layer "B.Cu") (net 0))
 (segment (start 125.325 112.165) (end 125.325 71.525) (width 0.25) (layer "B.Cu") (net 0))
 (segment (start 165.965 112.165) (end 165.965 71.525) (width 0.25) (layer "B.Cu") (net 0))
 (segment (start 206.732198 81.59) (end 203.51 81.59) (width 0.25) (layer "B.Cu") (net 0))
 (segment (start 149.86 67.31) (end 196.85 67.31) (width 0.25) (layer "B.Cu") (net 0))
 (segment (start 214.352198 80.05) (end 214.892198 80.59) (width 0.25) (layer "B.Cu") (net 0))
 (segment (start 196.85 66.04) (end 204.47 73.66) (width 0.25) (layer "B.Cu") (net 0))
 (segment (start 203.2 73.66) (end 203.2 80.01) (width 0.25) (layer "B.Cu") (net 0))
 (segment (start 219.162198 81.59) (end 217.162198 81.59) (width 0.25) (layer "B.Cu") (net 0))
 (segment (start 145.645 71.525) (end 149.86 67.31) (width 0.25) (layer "B.Cu") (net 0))
 (segment (start 204.47 78.74) (end 205.32 79.59) (width 0.25) (layer "B.Cu") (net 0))
 (segment (start 172.72 72.39) (end 171.855 71.525) (width 0.25) (layer "B.Cu") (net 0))
 (segment (start 130.81 66.04) (end 196.85 66.04) (width 0.25) (layer "B.Cu") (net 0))
 (segment (start 204.47 73.66) (end 204.47 78.74) (width 0.25) (layer "B.Cu") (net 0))
 (segment (start 230.107802 87.154396) (end 229.592198 87.67) (width 0.25) (layer "B.Cu") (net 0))
 (segment (start 172.72 77.47) (end 172.72 72.39) (width 0.25) (layer "B.Cu") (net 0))
 (segment (start 201.93 73.66) (end 198.12 69.85) (width 0.25) (layer "B.Cu") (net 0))
 (segment (start 171.855 71.525) (end 165.965 71.525) (width 0.25) (layer "B.Cu") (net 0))
 (segment (start 201.93 80.01) (end 201.93 73.66) (width 0.25) (layer "B.Cu") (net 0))
 (segment (start 198.12 69.85) (end 184.15 69.85) (width 0.25) (layer "B.Cu") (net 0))
 (segment (start 229.592198 87.67) (end 214.352198 87.67) (width 0.25) (layer "B.Cu") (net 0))
 (segment (start 203.2 80.01) (end 203.78 80.59) (width 0.25) (layer "B.Cu") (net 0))
 (segment (start 230.107802 84.82) (end 230.107802 87.154396) (width 0.25) (layer "B.Cu") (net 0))
 (segment (start 125.325 71.525) (end 130.81 66.04) (width 0.25) (layer "B.Cu") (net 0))
 (segment (start 145.645 71.525) (end 145.645 112.165) (width 0.25) (layer "B.Cu") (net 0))
 (segment (start 219.432198 83.86) (end 219.432198 81.32) (width 0.25) (layer "B.Cu") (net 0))
 (segment (start 230.107802 83.82) (end 219.472198 83.82) (width 0.25) (layer "B.Cu") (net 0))
 (segment (start 216.892198 81.59) (end 217.162198 81.59) (width 0.2) (layer "B.Cu") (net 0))
 (segment (start 214.892198 80.59) (end 216.892198 80.59) (width 0.25) (layer "B.Cu") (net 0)))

